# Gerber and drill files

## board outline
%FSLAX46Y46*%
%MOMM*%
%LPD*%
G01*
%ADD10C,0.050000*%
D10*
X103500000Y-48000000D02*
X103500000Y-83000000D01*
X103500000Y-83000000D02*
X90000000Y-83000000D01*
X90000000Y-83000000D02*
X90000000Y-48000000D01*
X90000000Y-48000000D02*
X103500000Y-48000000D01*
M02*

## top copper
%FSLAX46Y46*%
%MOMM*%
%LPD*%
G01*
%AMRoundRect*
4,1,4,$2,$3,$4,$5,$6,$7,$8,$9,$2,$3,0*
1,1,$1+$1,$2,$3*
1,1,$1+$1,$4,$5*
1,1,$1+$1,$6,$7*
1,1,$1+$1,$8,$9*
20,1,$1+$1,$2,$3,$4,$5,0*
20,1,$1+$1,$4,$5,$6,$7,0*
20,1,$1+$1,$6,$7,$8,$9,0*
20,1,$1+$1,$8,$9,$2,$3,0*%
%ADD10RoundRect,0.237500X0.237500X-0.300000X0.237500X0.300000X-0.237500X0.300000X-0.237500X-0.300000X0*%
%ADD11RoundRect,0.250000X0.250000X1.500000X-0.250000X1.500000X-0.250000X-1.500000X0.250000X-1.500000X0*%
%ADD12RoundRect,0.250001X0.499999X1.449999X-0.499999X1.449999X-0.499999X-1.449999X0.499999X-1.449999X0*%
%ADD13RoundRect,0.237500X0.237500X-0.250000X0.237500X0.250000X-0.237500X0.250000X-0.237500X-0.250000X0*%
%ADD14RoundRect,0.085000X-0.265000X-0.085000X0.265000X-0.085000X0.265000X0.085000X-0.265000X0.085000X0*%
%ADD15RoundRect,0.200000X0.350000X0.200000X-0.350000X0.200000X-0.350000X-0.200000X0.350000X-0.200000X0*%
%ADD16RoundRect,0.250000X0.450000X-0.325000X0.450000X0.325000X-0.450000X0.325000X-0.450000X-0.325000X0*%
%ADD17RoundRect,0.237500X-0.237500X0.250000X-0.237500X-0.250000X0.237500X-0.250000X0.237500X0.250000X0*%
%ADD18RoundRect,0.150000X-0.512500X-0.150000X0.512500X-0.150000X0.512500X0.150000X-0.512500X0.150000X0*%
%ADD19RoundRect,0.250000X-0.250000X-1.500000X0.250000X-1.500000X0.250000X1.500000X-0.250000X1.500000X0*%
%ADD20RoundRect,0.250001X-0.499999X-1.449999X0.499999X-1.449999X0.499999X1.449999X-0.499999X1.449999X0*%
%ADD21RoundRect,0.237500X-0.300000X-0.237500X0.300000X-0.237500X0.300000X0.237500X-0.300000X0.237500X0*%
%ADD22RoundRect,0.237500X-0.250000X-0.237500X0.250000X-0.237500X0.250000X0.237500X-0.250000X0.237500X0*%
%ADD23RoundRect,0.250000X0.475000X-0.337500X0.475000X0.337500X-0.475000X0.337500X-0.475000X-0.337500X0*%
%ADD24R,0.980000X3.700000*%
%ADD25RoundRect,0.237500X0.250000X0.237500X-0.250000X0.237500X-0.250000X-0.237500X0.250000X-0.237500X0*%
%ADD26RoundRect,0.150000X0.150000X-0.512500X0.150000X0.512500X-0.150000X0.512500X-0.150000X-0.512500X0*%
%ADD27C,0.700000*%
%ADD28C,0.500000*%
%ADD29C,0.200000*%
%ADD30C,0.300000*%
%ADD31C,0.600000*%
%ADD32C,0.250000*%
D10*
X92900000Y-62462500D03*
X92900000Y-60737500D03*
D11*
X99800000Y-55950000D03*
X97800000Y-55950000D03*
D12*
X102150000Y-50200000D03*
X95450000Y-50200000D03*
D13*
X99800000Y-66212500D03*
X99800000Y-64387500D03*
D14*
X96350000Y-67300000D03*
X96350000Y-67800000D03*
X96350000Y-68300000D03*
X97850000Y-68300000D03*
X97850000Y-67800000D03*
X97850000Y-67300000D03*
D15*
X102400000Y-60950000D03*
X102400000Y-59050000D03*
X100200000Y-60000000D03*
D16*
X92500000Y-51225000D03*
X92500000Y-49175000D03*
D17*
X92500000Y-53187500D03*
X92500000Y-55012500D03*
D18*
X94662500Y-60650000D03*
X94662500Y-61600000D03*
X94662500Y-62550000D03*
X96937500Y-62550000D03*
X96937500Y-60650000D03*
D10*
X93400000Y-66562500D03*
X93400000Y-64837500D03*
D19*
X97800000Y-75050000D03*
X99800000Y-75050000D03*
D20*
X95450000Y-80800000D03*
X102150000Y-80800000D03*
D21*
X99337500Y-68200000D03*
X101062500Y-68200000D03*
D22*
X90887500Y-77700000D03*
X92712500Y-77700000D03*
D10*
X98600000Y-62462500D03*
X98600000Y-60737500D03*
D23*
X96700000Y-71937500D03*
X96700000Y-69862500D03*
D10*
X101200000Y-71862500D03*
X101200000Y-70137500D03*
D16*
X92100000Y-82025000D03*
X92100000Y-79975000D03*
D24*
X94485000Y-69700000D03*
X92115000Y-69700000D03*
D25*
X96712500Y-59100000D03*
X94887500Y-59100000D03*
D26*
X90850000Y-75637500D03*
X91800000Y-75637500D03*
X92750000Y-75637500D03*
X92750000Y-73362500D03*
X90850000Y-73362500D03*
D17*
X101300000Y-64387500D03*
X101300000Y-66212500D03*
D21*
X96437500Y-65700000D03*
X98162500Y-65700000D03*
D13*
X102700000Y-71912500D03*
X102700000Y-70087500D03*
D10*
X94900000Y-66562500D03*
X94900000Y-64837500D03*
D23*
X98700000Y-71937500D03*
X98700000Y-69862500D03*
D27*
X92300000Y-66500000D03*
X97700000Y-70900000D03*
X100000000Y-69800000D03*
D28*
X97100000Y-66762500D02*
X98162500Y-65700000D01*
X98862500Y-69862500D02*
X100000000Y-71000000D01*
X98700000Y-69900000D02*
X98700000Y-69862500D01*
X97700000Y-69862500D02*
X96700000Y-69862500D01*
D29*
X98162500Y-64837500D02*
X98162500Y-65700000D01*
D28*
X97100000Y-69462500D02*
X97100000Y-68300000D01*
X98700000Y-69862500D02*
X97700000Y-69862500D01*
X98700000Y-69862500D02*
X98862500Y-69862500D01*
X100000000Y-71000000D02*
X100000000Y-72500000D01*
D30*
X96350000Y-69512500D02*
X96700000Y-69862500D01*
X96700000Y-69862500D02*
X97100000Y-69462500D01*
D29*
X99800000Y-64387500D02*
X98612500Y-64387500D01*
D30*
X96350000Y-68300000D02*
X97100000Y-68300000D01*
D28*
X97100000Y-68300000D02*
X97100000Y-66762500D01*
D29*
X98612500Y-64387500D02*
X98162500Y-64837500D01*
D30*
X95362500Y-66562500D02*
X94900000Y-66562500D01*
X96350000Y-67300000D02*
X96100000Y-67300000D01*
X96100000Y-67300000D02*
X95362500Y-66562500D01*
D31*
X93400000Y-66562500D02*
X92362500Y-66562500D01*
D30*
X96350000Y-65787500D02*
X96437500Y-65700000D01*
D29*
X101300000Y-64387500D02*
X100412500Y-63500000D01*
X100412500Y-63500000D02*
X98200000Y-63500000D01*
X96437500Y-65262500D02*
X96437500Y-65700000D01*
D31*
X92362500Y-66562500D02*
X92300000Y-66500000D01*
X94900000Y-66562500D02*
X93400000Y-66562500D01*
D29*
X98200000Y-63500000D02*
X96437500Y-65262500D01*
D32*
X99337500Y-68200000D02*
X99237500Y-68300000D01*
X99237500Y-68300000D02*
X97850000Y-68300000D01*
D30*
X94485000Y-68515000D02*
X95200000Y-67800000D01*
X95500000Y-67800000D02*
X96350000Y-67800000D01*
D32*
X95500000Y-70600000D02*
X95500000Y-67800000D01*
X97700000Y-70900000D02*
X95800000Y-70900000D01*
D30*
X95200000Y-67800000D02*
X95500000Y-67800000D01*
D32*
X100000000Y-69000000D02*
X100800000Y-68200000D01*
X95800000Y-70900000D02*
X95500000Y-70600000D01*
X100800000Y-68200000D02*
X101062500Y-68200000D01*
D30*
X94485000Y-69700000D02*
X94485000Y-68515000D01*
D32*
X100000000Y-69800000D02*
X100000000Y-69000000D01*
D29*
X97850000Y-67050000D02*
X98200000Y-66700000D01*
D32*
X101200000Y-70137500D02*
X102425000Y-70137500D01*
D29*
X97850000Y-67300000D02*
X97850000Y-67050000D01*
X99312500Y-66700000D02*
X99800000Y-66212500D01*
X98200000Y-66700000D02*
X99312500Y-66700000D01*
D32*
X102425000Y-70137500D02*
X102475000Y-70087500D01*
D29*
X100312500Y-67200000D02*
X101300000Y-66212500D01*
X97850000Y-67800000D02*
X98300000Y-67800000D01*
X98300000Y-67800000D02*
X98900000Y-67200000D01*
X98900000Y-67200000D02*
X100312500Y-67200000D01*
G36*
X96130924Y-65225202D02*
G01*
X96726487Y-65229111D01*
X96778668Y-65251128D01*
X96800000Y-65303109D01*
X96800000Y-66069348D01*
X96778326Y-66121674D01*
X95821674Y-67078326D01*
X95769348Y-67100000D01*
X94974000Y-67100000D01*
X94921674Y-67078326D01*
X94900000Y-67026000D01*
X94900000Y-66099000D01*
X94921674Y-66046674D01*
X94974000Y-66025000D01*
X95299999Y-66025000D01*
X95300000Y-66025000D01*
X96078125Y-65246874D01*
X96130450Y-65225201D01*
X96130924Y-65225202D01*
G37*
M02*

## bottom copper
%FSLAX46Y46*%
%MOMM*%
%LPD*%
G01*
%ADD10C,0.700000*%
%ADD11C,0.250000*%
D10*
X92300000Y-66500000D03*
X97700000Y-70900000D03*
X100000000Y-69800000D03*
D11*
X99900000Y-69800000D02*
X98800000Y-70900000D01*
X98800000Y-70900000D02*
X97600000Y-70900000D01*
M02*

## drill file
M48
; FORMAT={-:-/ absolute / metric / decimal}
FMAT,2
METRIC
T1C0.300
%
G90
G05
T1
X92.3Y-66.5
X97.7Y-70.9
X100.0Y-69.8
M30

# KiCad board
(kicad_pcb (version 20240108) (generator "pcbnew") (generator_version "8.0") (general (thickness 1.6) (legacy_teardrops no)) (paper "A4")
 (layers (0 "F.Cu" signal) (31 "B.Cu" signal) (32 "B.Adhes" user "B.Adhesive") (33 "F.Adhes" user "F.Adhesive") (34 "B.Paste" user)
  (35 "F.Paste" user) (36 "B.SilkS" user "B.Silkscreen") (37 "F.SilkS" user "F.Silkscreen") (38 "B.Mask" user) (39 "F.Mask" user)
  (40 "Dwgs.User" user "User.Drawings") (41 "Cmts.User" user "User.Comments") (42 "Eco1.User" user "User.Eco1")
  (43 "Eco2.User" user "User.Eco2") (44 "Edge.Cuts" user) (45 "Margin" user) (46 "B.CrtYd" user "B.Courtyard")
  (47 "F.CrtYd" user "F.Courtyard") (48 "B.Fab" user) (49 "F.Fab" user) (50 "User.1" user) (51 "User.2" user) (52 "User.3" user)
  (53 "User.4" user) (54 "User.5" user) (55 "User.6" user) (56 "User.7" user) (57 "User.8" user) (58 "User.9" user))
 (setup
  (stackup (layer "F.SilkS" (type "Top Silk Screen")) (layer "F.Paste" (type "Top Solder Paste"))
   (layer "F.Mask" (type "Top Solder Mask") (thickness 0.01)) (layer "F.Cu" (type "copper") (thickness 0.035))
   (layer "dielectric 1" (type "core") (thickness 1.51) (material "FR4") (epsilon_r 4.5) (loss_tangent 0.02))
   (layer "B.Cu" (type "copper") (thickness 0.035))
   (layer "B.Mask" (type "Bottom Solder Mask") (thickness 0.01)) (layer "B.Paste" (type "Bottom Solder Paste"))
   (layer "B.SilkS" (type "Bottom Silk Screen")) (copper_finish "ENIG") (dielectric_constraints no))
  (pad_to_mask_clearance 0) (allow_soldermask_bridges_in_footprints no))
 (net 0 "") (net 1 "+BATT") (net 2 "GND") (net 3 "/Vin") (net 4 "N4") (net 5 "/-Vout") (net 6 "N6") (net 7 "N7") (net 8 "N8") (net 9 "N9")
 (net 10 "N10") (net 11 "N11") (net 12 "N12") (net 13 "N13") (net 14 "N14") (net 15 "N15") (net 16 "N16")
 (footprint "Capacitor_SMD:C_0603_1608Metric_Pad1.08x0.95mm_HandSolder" (layer "F.Cu") (at 92.9 61.6 90)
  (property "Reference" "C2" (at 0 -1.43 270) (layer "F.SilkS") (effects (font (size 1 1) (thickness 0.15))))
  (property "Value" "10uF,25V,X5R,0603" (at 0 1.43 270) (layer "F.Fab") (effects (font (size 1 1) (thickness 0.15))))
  (pad "1" smd roundrect (at -0.8625 0 90) (size 1.075 0.95) (layers "F.Cu" "F.Paste" "F.Mask") (roundrect_rratio 0.25) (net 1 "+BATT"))
  (pad "2" smd roundrect (at 0.8625 0 90) (size 1.075 0.95) (layers "F.Cu" "F.Paste" "F.Mask") (roundrect_rratio 0.25) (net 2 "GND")))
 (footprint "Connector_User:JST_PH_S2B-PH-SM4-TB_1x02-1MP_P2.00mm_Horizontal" (layer "F.Cu") (at 98.8 53.1 180)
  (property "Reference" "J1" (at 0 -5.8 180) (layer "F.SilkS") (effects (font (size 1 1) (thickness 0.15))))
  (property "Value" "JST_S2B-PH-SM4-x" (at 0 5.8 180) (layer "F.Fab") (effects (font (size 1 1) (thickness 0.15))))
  (pad "1" smd roundrect (at -1 -2.85 180) (size 1 3.5) (layers "F.Cu" "F.Paste" "F.Mask") (roundrect_rratio 0.25) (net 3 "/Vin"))
  (pad "2" smd roundrect (at 1 -2.85 180) (size 1 3.5) (layers "F.Cu" "F.Paste" "F.Mask") (roundrect_rratio 0.25) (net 2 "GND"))
  (pad "MP1" smd roundrect (at -3.35 2.9 180) (size 1.5 3.4) (layers "F.Cu" "F.Paste" "F.Mask") (roundrect_rratio 0.166667) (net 2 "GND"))
  (pad "MP2" smd roundrect (at 3.35 2.9 180) (size 1.5 3.4) (layers "F.Cu" "F.Paste" "F.Mask") (roundrect_rratio 0.166667) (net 2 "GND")))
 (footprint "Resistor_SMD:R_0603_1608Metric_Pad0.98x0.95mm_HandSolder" (layer "F.Cu") (at 99.8 65.3 90)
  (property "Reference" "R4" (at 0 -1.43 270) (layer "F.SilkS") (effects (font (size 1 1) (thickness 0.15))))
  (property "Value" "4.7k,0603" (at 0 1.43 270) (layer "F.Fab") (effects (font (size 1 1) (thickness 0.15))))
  (pad "1" smd roundrect (at -0.9125 0 90) (size 0.975 0.95) (layers "F.Cu" "F.Paste" "F.Mask") (roundrect_rratio 0.25) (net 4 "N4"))
  (pad "2" smd roundrect (at 0.9125 0 90) (size 0.975 0.95) (layers "F.Cu" "F.Paste" "F.Mask") (roundrect_rratio 0.25) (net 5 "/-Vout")))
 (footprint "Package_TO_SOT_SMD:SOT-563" (layer "F.Cu") (at 97.1 67.8)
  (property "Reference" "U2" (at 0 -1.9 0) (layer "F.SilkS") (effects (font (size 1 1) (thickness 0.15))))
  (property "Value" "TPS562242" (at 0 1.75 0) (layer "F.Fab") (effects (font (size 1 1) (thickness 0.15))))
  (pad "1" smd roundrect (at -0.75 -0.5) (size 0.7 0.34) (layers "F.Cu" "F.Paste" "F.Mask") (roundrect_rratio 0.25) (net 1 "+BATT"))
  (pad "2" smd roundrect (at -0.75 0) (size 0.7 0.34) (layers "F.Cu" "F.Paste" "F.Mask") (roundrect_rratio 0.25) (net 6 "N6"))
  (pad "3" smd roundrect (at -0.75 0.5) (size 0.7 0.34) (layers "F.Cu" "F.Paste" "F.Mask") (roundrect_rratio 0.25) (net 5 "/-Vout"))
  (pad "4" smd roundrect (at 0.75 0.5) (size 0.7 0.34) (layers "F.Cu" "F.Paste" "F.Mask") (roundrect_rratio 0.25) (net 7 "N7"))
  (pad "5" smd roundrect (at 0.75 0) (size 0.7 0.34) (layers "F.Cu" "F.Paste" "F.Mask") (roundrect_rratio 0.25) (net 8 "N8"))
  (pad "6" smd roundrect (at 0.75 -0.5) (size 0.7 0.34) (layers "F.Cu" "F.Paste" "F.Mask") (roundrect_rratio 0.25) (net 4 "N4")))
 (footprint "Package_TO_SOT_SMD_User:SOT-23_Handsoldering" (layer "F.Cu") (at 101.3 60 180)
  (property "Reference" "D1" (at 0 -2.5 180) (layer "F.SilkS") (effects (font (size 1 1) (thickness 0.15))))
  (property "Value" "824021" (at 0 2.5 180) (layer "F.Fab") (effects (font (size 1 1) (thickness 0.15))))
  (pad "1" smd roundrect (at -1.1 -0.95 180) (size 1.1 0.8) (layers "F.Cu" "F.Paste" "F.Mask") (roundrect_rratio 0.25) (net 3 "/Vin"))
  (pad "2" smd roundrect (at -1.1 0.95 180) (size 1.1 0.8) (layers "F.Cu" "F.Paste" "F.Mask") (roundrect_rratio 0.25) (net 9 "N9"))
  (pad "3" smd roundrect (at 1.1 0 180) (size 1.1 0.8) (layers "F.Cu" "F.Paste" "F.Mask") (roundrect_rratio 0.25) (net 2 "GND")))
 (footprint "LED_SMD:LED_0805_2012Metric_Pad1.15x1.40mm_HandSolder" (layer "F.Cu") (at 92.5 50.2 90)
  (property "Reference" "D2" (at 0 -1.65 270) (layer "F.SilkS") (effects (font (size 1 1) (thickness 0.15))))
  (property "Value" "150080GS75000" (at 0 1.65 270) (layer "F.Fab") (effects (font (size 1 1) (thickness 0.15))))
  (pad "1" smd roundrect (at -1.025 0 90) (size 1.15 1.4) (layers "F.Cu" "F.Paste" "F.Mask") (roundrect_rratio 0.217391) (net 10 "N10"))
  (pad "2" smd roundrect (at 1.025 0 90) (size 1.15 1.4) (layers "F.Cu" "F.Paste" "F.Mask") (roundrect_rratio 0.217391) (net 3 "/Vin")))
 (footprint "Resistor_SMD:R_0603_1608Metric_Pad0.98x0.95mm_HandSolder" (layer "F.Cu") (at 92.5 54.1 -90)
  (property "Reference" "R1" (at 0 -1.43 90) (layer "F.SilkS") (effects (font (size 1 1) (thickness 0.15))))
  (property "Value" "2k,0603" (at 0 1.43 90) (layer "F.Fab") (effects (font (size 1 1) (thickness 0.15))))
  (pad "1" smd roundrect (at -0.9125 0 270) (size 0.975 0.95) (layers "F.Cu" "F.Paste" "F.Mask") (roundrect_rratio 0.25) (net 10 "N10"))
  (pad "2" smd roundrect (at 0.9125 0 270) (size 0.975 0.95) (layers "F.Cu" "F.Paste" "F.Mask") (roundrect_rratio 0.25) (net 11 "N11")))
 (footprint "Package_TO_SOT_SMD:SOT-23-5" (layer "F.Cu") (at 95.8 61.6)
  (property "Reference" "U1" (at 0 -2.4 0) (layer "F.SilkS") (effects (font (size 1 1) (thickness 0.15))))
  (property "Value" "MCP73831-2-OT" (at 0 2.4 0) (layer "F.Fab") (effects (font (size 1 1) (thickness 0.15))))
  (pad "1" smd roundrect (at -1.1375 -0.95) (size 1.325 0.6) (layers "F.Cu" "F.Paste" "F.Mask") (roundrect_rratio 0.25) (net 11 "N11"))
  (pad "2" smd roundrect (at -1.1375 0) (size 1.325 0.6) (layers "F.Cu" "F.Paste" "F.Mask") (roundrect_rratio 0.25) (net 2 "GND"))
  (pad "3" smd roundrect (at -1.1375 0.95) (size 1.325 0.6) (layers "F.Cu" "F.Paste" "F.Mask") (roundrect_rratio 0.25) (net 1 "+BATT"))
  (pad "4" smd roundrect (at 1.1375 0.95) (size 1.325 0.6) (layers "F.Cu" "F.Paste" "F.Mask") (roundrect_rratio 0.25) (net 3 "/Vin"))
  (pad "5" smd roundrect (at 1.1375 -0.95) (size 1.325 0.6) (layers "F.Cu" "F.Paste" "F.Mask") (roundrect_rratio 0.25) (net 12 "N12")))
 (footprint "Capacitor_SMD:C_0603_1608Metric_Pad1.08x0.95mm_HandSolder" (layer "F.Cu") (at 93.4 65.7 90)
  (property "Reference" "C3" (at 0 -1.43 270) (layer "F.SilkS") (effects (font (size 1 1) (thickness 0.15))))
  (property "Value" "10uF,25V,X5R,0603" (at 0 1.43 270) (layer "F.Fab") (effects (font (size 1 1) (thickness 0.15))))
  (pad "1" smd roundrect (at -0.8625 0 90) (size 1.075 0.95) (layers "F.Cu" "F.Paste" "F.Mask") (roundrect_rratio 0.25) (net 1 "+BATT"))
  (pad "2" smd roundrect (at 0.8625 0 90) (size 1.075 0.95) (layers "F.Cu" "F.Paste" "F.Mask") (roundrect_rratio 0.25) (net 2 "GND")))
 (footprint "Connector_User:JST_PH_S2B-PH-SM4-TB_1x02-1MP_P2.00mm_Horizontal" (layer "F.Cu") (at 98.8 77.9)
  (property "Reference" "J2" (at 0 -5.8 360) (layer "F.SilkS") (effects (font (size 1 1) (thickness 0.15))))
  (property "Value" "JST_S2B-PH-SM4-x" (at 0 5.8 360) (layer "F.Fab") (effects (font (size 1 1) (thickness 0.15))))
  (pad "1" smd roundrect (at -1 -2.85) (size 1 3.5) (layers "F.Cu" "F.Paste" "F.Mask") (roundrect_rratio 0.25) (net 2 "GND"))
  (pad "2" smd roundrect (at 1 -2.85) (size 1 3.5) (layers "F.Cu" "F.Paste" "F.Mask") (roundrect_rratio 0.25) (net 5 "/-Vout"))
  (pad "MP1" smd roundrect (at -3.35 2.9) (size 1.5 3.4) (layers "F.Cu" "F.Paste" "F.Mask") (roundrect_rratio 0.166667) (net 2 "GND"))
  (pad "MP2" smd roundrect (at 3.35 2.9) (size 1.5 3.4) (layers "F.Cu" "F.Paste" "F.Mask") (roundrect_rratio 0.166667) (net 2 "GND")))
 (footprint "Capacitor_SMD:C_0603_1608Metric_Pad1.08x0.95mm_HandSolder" (layer "F.Cu") (at 100.2 68.2)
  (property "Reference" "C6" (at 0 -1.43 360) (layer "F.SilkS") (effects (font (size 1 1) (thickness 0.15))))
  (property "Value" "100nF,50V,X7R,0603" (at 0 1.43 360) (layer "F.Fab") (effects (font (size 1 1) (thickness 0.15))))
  (pad "1" smd roundrect (at -0.8625 0) (size 1.075 0.95) (layers "F.Cu" "F.Paste" "F.Mask") (roundrect_rratio 0.25) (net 7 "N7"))
  (pad "2" smd roundrect (at 0.8625 0) (size 1.075 0.95) (layers "F.Cu" "F.Paste" "F.Mask") (roundrect_rratio 0.25) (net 6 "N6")))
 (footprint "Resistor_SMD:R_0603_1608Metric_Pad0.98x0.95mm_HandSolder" (layer "F.Cu") (at 91.8 77.7)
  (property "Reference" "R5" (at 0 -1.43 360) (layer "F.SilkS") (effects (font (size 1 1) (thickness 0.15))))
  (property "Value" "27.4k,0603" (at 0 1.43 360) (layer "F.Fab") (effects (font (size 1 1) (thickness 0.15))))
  (pad "1" smd roundrect (at -0.9125 0) (size 0.975 0.95) (layers "F.Cu" "F.Paste" "F.Mask") (roundrect_rratio 0.25) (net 1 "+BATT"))
  (pad "2" smd roundrect (at 0.9125 0) (size 0.975 0.95) (layers "F.Cu" "F.Paste" "F.Mask") (roundrect_rratio 0.25) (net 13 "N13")))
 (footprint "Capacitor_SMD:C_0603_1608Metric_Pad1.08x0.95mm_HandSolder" (layer "F.Cu") (at 98.6 61.6 90)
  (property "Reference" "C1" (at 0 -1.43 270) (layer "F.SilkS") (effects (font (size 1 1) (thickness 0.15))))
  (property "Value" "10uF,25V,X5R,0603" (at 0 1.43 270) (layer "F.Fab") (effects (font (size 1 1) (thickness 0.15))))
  (pad "1" smd roundrect (at -0.8625 0 90) (size 1.075 0.95) (layers "F.Cu" "F.Paste" "F.Mask") (roundrect_rratio 0.25) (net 3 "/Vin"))
  (pad "2" smd roundrect (at 0.8625 0 90) (size 1.075 0.95) (layers "F.Cu" "F.Paste" "F.Mask") (roundrect_rratio 0.25) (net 2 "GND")))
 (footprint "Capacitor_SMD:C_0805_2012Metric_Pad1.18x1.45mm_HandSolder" (layer "F.Cu") (at 96.7 70.9 90)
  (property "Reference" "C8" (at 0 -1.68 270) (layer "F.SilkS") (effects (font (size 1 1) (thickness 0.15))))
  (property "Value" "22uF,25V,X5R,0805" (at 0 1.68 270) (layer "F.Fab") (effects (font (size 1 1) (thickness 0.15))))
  (pad "1" smd roundrect (at -1.0375 0 90) (size 1.175 1.45) (layers "F.Cu" "F.Paste" "F.Mask") (roundrect_rratio 0.212766) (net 2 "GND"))
  (pad "2" smd roundrect (at 1.0375 0 90) (size 1.175 1.45) (layers "F.Cu" "F.Paste" "F.Mask") (roundrect_rratio 0.212766) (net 5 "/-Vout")))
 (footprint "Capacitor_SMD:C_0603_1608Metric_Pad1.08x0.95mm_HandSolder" (layer "F.Cu") (at 101.2 71 90)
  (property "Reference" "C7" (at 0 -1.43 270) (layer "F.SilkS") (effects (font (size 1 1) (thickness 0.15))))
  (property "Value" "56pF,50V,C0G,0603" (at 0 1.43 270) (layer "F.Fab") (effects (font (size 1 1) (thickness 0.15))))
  (pad "1" smd roundrect (at -0.8625 0 90) (size 1.075 0.95) (layers "F.Cu" "F.Paste" "F.Mask") (roundrect_rratio 0.25) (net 2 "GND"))
  (pad "2" smd roundrect (at 0.8625 0 90) (size 1.075 0.95) (layers "F.Cu" "F.Paste" "F.Mask") (roundrect_rratio 0.25) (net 4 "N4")))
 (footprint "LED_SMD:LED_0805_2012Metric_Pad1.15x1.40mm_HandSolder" (layer "F.Cu") (at 92.1 81 90)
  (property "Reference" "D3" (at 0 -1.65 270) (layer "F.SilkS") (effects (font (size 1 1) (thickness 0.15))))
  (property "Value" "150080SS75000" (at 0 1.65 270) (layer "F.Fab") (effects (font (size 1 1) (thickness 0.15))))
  (pad "1" smd roundrect (at -1.025 0 90) (size 1.15 1.4) (layers "F.Cu" "F.Paste" "F.Mask") (roundrect_rratio 0.217391) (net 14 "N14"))
  (pad "2" smd roundrect (at 1.025 0 90) (size 1.15 1.4) (layers "F.Cu" "F.Paste" "F.Mask") (roundrect_rratio 0.217391) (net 13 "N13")))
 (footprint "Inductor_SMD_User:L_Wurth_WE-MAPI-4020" (layer "F.Cu") (at 93.3 69.7 180)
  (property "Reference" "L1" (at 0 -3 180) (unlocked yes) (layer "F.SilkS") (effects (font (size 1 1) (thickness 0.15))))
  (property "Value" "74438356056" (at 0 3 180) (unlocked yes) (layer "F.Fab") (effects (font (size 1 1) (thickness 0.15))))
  (pad "1" smd rect (at -1.185 0 180) (size 0.98 3.7) (layers "F.Cu" "F.Paste" "F.Mask") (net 6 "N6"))
  (pad "2" smd rect (at 1.185 0 180) (size 0.98 3.7) (layers "F.Cu" "F.Paste" "F.Mask") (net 2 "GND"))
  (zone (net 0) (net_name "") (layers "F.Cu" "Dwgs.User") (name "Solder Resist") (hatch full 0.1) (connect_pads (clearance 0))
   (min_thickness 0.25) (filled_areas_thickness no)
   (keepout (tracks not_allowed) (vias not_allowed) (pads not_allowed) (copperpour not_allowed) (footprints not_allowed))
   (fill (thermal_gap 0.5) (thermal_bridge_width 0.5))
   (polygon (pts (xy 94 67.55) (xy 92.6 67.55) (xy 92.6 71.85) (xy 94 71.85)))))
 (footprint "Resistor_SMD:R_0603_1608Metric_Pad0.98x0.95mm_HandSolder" (layer "F.Cu") (at 95.8 59.1 180)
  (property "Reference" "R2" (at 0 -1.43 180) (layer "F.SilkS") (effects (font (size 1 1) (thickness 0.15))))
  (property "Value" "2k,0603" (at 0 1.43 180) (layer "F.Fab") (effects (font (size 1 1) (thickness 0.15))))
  (pad "1" smd roundrect (at -0.9125 0 180) (size 0.975 0.95) (layers "F.Cu" "F.Paste" "F.Mask") (roundrect_rratio 0.25) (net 12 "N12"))
  (pad "2" smd roundrect (at 0.9125 0 180) (size 0.975 0.95) (layers "F.Cu" "F.Paste" "F.Mask") (roundrect_rratio 0.25) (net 2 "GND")))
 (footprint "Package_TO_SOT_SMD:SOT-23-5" (layer "F.Cu") (at 91.8 74.5 90)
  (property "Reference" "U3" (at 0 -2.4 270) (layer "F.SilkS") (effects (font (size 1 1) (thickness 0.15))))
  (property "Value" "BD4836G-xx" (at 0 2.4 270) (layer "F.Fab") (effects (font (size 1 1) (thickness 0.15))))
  (pad "1" smd roundrect (at -1.1375 -0.95 90) (size 1.325 0.6) (layers "F.Cu" "F.Paste" "F.Mask") (roundrect_rratio 0.25) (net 14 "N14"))
  (pad "2" smd roundrect (at -1.1375 0 90) (size 1.325 0.6) (layers "F.Cu" "F.Paste" "F.Mask") (roundrect_rratio 0.25) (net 1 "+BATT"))
  (pad "3" smd roundrect (at -1.1375 0.95 90) (size 1.325 0.6) (layers "F.Cu" "F.Paste" "F.Mask") (roundrect_rratio 0.25) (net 2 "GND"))
  (pad "4" smd roundrect (at 1.1375 0.95 90) (size 1.325 0.6) (layers "F.Cu" "F.Paste" "F.Mask") (roundrect_rratio 0.25) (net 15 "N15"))
  (pad "5" smd roundrect (at 1.1375 -0.95 90) (size 1.325 0.6) (layers "F.Cu" "F.Paste" "F.Mask") (roundrect_rratio 0.25) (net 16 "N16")))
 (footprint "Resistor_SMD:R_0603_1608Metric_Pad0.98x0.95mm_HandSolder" (layer "F.Cu") (at 101.3 65.3 -90)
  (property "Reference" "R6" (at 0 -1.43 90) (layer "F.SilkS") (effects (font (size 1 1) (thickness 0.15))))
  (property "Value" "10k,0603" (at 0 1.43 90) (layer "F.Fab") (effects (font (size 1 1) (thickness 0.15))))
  (pad "1" smd roundrect (at -0.9125 0 270) (size 0.975 0.95) (layers "F.Cu" "F.Paste" "F.Mask") (roundrect_rratio 0.25) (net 1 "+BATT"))
  (pad "2" smd roundrect (at 0.9125 0 270) (size 0.975 0.95) (layers "F.Cu" "F.Paste" "F.Mask") (roundrect_rratio 0.25) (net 8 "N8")))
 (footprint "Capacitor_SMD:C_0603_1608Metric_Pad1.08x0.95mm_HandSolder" (layer "F.Cu") (at 97.3 65.7)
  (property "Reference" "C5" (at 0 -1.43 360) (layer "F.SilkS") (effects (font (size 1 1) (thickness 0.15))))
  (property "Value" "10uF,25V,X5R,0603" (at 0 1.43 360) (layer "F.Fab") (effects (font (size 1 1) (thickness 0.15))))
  (pad "1" smd roundrect (at -0.8625 0) (size 1.075 0.95) (layers "F.Cu" "F.Paste" "F.Mask") (roundrect_rratio 0.25) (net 1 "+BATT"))
  (pad "2" smd roundrect (at 0.8625 0) (size 1.075 0.95) (layers "F.Cu" "F.Paste" "F.Mask") (roundrect_rratio 0.25) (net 5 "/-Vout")))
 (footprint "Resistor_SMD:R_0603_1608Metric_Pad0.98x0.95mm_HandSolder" (layer "F.Cu") (at 102.7 71 90)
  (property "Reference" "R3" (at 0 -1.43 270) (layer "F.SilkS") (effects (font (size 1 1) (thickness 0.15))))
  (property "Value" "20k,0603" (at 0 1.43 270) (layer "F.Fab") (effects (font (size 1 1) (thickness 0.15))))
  (pad "1" smd roundrect (at -0.9125 0 90) (size 0.975 0.95) (layers "F.Cu" "F.Paste" "F.Mask") (roundrect_rratio 0.25) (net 2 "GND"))
  (pad "2" smd roundrect (at 0.9125 0 90) (size 0.975 0.95) (layers "F.Cu" "F.Paste" "F.Mask") (roundrect_rratio 0.25) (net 4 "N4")))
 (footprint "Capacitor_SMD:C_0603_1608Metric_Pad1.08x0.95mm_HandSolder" (layer "F.Cu") (at 94.9 65.7 90)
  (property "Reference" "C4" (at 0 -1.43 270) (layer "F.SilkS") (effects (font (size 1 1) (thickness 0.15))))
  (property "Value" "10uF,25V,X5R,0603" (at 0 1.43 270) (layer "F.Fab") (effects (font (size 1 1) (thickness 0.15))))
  (pad "1" smd roundrect (at -0.8625 0 90) (size 1.075 0.95) (layers "F.Cu" "F.Paste" "F.Mask") (roundrect_rratio 0.25) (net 1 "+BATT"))
  (pad "2" smd roundrect (at 0.8625 0 90) (size 1.075 0.95) (layers "F.Cu" "F.Paste" "F.Mask") (roundrect_rratio 0.25) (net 2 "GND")))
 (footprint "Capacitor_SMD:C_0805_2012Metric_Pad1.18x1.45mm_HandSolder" (layer "F.Cu") (at 98.7 70.9 90)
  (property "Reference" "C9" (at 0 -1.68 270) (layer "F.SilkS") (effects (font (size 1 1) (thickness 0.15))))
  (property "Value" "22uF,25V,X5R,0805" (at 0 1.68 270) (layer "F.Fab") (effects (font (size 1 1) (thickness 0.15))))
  (pad "1" smd roundrect (at -1.0375 0 90) (size 1.175 1.45) (layers "F.Cu" "F.Paste" "F.Mask") (roundrect_rratio 0.212766) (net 2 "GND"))
  (pad "2" smd roundrect (at 1.0375 0 90) (size 1.175 1.45) (layers "F.Cu" "F.Paste" "F.Mask") (roundrect_rratio 0.212766) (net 5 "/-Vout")))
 (gr_line (start 103.5 48) (end 103.5 83) (stroke (width 0.05) (type default)) (layer "Edge.Cuts"))
 (gr_line (start 103.5 83) (end 90 83) (stroke (width 0.05) (type default)) (layer "Edge.Cuts"))
 (gr_line (start 90 83) (end 90 48) (stroke (width 0.05) (type default)) (layer "Edge.Cuts"))
 (gr_line (start 90 48) (end 103.5 48) (stroke (width 0.05) (type default)) (layer "Edge.Cuts"))
 (segment (start 97.1 66.7625) (end 98.1625 65.7) (width 0.5) (layer "F.Cu") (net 5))
 (segment (start 98.8625 69.8625) (end 100 71) (width 0.5) (layer "F.Cu") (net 5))
 (segment (start 98.7 69.9) (end 98.7 69.8625) (width 0.5) (layer "F.Cu") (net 5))
 (segment (start 97.7 69.8625) (end 96.7 69.8625) (width 0.5) (layer "F.Cu") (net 5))
 (segment (start 98.1625 64.8375) (end 98.1625 65.7) (width 0.2) (layer "F.Cu") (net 5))
 (segment (start 97.1 69.4625) (end 97.1 68.3) (width 0.5) (layer "F.Cu") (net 5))
 (segment (start 98.7 69.8625) (end 97.7 69.8625) (width 0.5) (layer "F.Cu") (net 5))
 (segment (start 98.7 69.8625) (end 98.8625 69.8625) (width 0.5) (layer "F.Cu") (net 5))
 (segment (start 100 71) (end 100 72.5) (width 0.5) (layer "F.Cu") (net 5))
 (segment (start 96.35 69.5125) (end 96.7 69.8625) (width 0.3) (layer "F.Cu") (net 5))
 (segment (start 96.7 69.8625) (end 97.1 69.4625) (width 0.3) (layer "F.Cu") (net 5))
 (segment (start 99.8 64.3875) (end 98.6125 64.3875) (width 0.2) (layer "F.Cu") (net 5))
 (segment (start 96.35 68.3) (end 97.1 68.3) (width 0.3) (layer "F.Cu") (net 5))
 (segment (start 97.1 68.3) (end 97.1 66.7625) (width 0.5) (layer "F.Cu") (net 5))
 (segment (start 98.6125 64.3875) (end 98.1625 64.8375) (width 0.2) (layer "F.Cu") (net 5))
 (segment (start 95.3625 66.5625) (end 94.9 66.5625) (width 0.3) (layer "F.Cu") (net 1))
 (segment (start 96.35 67.3) (end 96.1 67.3) (width 0.3) (layer "F.Cu") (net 1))
 (segment (start 96.1 67.3) (end 95.3625 66.5625) (width 0.3) (layer "F.Cu") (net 1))
 (segment (start 93.4 66.5625) (end 92.3625 66.5625) (width 0.6) (layer "F.Cu") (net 1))
 (segment (start 96.35 65.7875) (end 96.4375 65.7) (width 0.3) (layer "F.Cu") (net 1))
 (segment (start 101.3 64.3875) (end 100.4125 63.5) (width 0.2) (layer "F.Cu") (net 1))
 (segment (start 100.4125 63.5) (end 98.2 63.5) (width 0.2) (layer "F.Cu") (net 1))
 (segment (start 96.4375 65.2625) (end 96.4375 65.7) (width 0.2) (layer "F.Cu") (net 1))
 (segment (start 92.3625 66.5625) (end 92.3 66.5) (width 0.6) (layer "F.Cu") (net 1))
 (segment (start 94.9 66.5625) (end 93.4 66.5625) (width 0.6) (layer "F.Cu") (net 1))
 (segment (start 98.2 63.5) (end 96.4375 65.2625) (width 0.2) (layer "F.Cu") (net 1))
 (via (at 92.3 66.5) (size 0.7) (drill 0.3) (layers "F.Cu" "B.Cu") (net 1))
 (segment (start 99.3375 68.2) (end 99.2375 68.3) (width 0.25) (layer "F.Cu") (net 7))
 (segment (start 99.2375 68.3) (end 97.85 68.3) (width 0.25) (layer "F.Cu") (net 7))
 (segment (start 94.485 68.515) (end 95.2 67.8) (width 0.3) (layer "F.Cu") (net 6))
 (segment (start 95.5 67.8) (end 96.35 67.8) (width 0.3) (layer "F.Cu") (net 6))
 (segment (start 95.5 70.6) (end 95.5 67.8) (width 0.25) (layer "F.Cu") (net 6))
 (segment (start 97.7 70.9) (end 95.8 70.9) (width 0.25) (layer "F.Cu") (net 6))
 (segment (start 95.2 67.8) (end 95.5 67.8) (width 0.3) (layer "F.Cu") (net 6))
 (segment (start 100 69) (end 100.8 68.2) (width 0.25) (layer "F.Cu") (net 6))
 (segment (start 95.8 70.9) (end 95.5 70.6) (width 0.25) (layer "F.Cu") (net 6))
 (segment (start 100.8 68.2) (end 101.0625 68.2) (width 0.25) (layer "F.Cu") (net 6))
 (segment (start 94.485 69.7) (end 94.485 68.515) (width 0.3) (layer "F.Cu") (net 6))
 (segment (start 100 69.8) (end 100 69) (width 0.25) (layer "F.Cu") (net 6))
 (via (at 97.7 70.9) (size 0.7) (drill 0.3) (layers "F.Cu" "B.Cu") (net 6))
 (via (at 100 69.8) (size 0.7) (drill 0.3) (layers "F.Cu" "B.Cu") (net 6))
 (segment (start 99.9 69.8) (end 98.8 70.9) (width 0.25) (layer "B.Cu") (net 6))
 (segment (start 98.8 70.9) (end 97.6 70.9) (width 0.25) (layer "B.Cu") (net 6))
 (segment (start 97.85 67.05) (end 98.2 66.7) (width 0.2) (layer "F.Cu") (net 4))
 (segment (start 101.2 70.1375) (end 102.425 70.1375) (width 0.25) (layer "F.Cu") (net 4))
 (segment (start 97.85 67.3) (end 97.85 67.05) (width 0.2) (layer "F.Cu") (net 4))
 (segment (start 99.3125 66.7) (end 99.8 66.2125) (width 0.2) (layer "F.Cu") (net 4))
 (segment (start 98.2 66.7) (end 99.3125 66.7) (width 0.2) (layer "F.Cu") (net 4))
 (segment (start 102.425 70.1375) (end 102.475 70.0875) (width 0.25) (layer "F.Cu") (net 4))
 (segment (start 100.3125 67.2) (end 101.3 66.2125) (width 0.2) (layer "F.Cu") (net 8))
 (segment (start 97.85 67.8) (end 98.3 67.8) (width 0.2) (layer "F.Cu") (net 8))
 (segment (start 98.3 67.8) (end 98.9 67.2) (width 0.2) (layer "F.Cu") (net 8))
 (segment (start 98.9 67.2) (end 100.3125 67.2) (width 0.2) (layer "F.Cu") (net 8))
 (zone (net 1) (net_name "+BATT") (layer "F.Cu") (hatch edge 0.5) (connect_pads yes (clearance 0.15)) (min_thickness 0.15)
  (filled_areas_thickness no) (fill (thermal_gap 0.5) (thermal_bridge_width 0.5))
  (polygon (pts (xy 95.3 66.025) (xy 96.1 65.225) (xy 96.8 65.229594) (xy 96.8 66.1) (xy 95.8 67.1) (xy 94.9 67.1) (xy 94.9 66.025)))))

